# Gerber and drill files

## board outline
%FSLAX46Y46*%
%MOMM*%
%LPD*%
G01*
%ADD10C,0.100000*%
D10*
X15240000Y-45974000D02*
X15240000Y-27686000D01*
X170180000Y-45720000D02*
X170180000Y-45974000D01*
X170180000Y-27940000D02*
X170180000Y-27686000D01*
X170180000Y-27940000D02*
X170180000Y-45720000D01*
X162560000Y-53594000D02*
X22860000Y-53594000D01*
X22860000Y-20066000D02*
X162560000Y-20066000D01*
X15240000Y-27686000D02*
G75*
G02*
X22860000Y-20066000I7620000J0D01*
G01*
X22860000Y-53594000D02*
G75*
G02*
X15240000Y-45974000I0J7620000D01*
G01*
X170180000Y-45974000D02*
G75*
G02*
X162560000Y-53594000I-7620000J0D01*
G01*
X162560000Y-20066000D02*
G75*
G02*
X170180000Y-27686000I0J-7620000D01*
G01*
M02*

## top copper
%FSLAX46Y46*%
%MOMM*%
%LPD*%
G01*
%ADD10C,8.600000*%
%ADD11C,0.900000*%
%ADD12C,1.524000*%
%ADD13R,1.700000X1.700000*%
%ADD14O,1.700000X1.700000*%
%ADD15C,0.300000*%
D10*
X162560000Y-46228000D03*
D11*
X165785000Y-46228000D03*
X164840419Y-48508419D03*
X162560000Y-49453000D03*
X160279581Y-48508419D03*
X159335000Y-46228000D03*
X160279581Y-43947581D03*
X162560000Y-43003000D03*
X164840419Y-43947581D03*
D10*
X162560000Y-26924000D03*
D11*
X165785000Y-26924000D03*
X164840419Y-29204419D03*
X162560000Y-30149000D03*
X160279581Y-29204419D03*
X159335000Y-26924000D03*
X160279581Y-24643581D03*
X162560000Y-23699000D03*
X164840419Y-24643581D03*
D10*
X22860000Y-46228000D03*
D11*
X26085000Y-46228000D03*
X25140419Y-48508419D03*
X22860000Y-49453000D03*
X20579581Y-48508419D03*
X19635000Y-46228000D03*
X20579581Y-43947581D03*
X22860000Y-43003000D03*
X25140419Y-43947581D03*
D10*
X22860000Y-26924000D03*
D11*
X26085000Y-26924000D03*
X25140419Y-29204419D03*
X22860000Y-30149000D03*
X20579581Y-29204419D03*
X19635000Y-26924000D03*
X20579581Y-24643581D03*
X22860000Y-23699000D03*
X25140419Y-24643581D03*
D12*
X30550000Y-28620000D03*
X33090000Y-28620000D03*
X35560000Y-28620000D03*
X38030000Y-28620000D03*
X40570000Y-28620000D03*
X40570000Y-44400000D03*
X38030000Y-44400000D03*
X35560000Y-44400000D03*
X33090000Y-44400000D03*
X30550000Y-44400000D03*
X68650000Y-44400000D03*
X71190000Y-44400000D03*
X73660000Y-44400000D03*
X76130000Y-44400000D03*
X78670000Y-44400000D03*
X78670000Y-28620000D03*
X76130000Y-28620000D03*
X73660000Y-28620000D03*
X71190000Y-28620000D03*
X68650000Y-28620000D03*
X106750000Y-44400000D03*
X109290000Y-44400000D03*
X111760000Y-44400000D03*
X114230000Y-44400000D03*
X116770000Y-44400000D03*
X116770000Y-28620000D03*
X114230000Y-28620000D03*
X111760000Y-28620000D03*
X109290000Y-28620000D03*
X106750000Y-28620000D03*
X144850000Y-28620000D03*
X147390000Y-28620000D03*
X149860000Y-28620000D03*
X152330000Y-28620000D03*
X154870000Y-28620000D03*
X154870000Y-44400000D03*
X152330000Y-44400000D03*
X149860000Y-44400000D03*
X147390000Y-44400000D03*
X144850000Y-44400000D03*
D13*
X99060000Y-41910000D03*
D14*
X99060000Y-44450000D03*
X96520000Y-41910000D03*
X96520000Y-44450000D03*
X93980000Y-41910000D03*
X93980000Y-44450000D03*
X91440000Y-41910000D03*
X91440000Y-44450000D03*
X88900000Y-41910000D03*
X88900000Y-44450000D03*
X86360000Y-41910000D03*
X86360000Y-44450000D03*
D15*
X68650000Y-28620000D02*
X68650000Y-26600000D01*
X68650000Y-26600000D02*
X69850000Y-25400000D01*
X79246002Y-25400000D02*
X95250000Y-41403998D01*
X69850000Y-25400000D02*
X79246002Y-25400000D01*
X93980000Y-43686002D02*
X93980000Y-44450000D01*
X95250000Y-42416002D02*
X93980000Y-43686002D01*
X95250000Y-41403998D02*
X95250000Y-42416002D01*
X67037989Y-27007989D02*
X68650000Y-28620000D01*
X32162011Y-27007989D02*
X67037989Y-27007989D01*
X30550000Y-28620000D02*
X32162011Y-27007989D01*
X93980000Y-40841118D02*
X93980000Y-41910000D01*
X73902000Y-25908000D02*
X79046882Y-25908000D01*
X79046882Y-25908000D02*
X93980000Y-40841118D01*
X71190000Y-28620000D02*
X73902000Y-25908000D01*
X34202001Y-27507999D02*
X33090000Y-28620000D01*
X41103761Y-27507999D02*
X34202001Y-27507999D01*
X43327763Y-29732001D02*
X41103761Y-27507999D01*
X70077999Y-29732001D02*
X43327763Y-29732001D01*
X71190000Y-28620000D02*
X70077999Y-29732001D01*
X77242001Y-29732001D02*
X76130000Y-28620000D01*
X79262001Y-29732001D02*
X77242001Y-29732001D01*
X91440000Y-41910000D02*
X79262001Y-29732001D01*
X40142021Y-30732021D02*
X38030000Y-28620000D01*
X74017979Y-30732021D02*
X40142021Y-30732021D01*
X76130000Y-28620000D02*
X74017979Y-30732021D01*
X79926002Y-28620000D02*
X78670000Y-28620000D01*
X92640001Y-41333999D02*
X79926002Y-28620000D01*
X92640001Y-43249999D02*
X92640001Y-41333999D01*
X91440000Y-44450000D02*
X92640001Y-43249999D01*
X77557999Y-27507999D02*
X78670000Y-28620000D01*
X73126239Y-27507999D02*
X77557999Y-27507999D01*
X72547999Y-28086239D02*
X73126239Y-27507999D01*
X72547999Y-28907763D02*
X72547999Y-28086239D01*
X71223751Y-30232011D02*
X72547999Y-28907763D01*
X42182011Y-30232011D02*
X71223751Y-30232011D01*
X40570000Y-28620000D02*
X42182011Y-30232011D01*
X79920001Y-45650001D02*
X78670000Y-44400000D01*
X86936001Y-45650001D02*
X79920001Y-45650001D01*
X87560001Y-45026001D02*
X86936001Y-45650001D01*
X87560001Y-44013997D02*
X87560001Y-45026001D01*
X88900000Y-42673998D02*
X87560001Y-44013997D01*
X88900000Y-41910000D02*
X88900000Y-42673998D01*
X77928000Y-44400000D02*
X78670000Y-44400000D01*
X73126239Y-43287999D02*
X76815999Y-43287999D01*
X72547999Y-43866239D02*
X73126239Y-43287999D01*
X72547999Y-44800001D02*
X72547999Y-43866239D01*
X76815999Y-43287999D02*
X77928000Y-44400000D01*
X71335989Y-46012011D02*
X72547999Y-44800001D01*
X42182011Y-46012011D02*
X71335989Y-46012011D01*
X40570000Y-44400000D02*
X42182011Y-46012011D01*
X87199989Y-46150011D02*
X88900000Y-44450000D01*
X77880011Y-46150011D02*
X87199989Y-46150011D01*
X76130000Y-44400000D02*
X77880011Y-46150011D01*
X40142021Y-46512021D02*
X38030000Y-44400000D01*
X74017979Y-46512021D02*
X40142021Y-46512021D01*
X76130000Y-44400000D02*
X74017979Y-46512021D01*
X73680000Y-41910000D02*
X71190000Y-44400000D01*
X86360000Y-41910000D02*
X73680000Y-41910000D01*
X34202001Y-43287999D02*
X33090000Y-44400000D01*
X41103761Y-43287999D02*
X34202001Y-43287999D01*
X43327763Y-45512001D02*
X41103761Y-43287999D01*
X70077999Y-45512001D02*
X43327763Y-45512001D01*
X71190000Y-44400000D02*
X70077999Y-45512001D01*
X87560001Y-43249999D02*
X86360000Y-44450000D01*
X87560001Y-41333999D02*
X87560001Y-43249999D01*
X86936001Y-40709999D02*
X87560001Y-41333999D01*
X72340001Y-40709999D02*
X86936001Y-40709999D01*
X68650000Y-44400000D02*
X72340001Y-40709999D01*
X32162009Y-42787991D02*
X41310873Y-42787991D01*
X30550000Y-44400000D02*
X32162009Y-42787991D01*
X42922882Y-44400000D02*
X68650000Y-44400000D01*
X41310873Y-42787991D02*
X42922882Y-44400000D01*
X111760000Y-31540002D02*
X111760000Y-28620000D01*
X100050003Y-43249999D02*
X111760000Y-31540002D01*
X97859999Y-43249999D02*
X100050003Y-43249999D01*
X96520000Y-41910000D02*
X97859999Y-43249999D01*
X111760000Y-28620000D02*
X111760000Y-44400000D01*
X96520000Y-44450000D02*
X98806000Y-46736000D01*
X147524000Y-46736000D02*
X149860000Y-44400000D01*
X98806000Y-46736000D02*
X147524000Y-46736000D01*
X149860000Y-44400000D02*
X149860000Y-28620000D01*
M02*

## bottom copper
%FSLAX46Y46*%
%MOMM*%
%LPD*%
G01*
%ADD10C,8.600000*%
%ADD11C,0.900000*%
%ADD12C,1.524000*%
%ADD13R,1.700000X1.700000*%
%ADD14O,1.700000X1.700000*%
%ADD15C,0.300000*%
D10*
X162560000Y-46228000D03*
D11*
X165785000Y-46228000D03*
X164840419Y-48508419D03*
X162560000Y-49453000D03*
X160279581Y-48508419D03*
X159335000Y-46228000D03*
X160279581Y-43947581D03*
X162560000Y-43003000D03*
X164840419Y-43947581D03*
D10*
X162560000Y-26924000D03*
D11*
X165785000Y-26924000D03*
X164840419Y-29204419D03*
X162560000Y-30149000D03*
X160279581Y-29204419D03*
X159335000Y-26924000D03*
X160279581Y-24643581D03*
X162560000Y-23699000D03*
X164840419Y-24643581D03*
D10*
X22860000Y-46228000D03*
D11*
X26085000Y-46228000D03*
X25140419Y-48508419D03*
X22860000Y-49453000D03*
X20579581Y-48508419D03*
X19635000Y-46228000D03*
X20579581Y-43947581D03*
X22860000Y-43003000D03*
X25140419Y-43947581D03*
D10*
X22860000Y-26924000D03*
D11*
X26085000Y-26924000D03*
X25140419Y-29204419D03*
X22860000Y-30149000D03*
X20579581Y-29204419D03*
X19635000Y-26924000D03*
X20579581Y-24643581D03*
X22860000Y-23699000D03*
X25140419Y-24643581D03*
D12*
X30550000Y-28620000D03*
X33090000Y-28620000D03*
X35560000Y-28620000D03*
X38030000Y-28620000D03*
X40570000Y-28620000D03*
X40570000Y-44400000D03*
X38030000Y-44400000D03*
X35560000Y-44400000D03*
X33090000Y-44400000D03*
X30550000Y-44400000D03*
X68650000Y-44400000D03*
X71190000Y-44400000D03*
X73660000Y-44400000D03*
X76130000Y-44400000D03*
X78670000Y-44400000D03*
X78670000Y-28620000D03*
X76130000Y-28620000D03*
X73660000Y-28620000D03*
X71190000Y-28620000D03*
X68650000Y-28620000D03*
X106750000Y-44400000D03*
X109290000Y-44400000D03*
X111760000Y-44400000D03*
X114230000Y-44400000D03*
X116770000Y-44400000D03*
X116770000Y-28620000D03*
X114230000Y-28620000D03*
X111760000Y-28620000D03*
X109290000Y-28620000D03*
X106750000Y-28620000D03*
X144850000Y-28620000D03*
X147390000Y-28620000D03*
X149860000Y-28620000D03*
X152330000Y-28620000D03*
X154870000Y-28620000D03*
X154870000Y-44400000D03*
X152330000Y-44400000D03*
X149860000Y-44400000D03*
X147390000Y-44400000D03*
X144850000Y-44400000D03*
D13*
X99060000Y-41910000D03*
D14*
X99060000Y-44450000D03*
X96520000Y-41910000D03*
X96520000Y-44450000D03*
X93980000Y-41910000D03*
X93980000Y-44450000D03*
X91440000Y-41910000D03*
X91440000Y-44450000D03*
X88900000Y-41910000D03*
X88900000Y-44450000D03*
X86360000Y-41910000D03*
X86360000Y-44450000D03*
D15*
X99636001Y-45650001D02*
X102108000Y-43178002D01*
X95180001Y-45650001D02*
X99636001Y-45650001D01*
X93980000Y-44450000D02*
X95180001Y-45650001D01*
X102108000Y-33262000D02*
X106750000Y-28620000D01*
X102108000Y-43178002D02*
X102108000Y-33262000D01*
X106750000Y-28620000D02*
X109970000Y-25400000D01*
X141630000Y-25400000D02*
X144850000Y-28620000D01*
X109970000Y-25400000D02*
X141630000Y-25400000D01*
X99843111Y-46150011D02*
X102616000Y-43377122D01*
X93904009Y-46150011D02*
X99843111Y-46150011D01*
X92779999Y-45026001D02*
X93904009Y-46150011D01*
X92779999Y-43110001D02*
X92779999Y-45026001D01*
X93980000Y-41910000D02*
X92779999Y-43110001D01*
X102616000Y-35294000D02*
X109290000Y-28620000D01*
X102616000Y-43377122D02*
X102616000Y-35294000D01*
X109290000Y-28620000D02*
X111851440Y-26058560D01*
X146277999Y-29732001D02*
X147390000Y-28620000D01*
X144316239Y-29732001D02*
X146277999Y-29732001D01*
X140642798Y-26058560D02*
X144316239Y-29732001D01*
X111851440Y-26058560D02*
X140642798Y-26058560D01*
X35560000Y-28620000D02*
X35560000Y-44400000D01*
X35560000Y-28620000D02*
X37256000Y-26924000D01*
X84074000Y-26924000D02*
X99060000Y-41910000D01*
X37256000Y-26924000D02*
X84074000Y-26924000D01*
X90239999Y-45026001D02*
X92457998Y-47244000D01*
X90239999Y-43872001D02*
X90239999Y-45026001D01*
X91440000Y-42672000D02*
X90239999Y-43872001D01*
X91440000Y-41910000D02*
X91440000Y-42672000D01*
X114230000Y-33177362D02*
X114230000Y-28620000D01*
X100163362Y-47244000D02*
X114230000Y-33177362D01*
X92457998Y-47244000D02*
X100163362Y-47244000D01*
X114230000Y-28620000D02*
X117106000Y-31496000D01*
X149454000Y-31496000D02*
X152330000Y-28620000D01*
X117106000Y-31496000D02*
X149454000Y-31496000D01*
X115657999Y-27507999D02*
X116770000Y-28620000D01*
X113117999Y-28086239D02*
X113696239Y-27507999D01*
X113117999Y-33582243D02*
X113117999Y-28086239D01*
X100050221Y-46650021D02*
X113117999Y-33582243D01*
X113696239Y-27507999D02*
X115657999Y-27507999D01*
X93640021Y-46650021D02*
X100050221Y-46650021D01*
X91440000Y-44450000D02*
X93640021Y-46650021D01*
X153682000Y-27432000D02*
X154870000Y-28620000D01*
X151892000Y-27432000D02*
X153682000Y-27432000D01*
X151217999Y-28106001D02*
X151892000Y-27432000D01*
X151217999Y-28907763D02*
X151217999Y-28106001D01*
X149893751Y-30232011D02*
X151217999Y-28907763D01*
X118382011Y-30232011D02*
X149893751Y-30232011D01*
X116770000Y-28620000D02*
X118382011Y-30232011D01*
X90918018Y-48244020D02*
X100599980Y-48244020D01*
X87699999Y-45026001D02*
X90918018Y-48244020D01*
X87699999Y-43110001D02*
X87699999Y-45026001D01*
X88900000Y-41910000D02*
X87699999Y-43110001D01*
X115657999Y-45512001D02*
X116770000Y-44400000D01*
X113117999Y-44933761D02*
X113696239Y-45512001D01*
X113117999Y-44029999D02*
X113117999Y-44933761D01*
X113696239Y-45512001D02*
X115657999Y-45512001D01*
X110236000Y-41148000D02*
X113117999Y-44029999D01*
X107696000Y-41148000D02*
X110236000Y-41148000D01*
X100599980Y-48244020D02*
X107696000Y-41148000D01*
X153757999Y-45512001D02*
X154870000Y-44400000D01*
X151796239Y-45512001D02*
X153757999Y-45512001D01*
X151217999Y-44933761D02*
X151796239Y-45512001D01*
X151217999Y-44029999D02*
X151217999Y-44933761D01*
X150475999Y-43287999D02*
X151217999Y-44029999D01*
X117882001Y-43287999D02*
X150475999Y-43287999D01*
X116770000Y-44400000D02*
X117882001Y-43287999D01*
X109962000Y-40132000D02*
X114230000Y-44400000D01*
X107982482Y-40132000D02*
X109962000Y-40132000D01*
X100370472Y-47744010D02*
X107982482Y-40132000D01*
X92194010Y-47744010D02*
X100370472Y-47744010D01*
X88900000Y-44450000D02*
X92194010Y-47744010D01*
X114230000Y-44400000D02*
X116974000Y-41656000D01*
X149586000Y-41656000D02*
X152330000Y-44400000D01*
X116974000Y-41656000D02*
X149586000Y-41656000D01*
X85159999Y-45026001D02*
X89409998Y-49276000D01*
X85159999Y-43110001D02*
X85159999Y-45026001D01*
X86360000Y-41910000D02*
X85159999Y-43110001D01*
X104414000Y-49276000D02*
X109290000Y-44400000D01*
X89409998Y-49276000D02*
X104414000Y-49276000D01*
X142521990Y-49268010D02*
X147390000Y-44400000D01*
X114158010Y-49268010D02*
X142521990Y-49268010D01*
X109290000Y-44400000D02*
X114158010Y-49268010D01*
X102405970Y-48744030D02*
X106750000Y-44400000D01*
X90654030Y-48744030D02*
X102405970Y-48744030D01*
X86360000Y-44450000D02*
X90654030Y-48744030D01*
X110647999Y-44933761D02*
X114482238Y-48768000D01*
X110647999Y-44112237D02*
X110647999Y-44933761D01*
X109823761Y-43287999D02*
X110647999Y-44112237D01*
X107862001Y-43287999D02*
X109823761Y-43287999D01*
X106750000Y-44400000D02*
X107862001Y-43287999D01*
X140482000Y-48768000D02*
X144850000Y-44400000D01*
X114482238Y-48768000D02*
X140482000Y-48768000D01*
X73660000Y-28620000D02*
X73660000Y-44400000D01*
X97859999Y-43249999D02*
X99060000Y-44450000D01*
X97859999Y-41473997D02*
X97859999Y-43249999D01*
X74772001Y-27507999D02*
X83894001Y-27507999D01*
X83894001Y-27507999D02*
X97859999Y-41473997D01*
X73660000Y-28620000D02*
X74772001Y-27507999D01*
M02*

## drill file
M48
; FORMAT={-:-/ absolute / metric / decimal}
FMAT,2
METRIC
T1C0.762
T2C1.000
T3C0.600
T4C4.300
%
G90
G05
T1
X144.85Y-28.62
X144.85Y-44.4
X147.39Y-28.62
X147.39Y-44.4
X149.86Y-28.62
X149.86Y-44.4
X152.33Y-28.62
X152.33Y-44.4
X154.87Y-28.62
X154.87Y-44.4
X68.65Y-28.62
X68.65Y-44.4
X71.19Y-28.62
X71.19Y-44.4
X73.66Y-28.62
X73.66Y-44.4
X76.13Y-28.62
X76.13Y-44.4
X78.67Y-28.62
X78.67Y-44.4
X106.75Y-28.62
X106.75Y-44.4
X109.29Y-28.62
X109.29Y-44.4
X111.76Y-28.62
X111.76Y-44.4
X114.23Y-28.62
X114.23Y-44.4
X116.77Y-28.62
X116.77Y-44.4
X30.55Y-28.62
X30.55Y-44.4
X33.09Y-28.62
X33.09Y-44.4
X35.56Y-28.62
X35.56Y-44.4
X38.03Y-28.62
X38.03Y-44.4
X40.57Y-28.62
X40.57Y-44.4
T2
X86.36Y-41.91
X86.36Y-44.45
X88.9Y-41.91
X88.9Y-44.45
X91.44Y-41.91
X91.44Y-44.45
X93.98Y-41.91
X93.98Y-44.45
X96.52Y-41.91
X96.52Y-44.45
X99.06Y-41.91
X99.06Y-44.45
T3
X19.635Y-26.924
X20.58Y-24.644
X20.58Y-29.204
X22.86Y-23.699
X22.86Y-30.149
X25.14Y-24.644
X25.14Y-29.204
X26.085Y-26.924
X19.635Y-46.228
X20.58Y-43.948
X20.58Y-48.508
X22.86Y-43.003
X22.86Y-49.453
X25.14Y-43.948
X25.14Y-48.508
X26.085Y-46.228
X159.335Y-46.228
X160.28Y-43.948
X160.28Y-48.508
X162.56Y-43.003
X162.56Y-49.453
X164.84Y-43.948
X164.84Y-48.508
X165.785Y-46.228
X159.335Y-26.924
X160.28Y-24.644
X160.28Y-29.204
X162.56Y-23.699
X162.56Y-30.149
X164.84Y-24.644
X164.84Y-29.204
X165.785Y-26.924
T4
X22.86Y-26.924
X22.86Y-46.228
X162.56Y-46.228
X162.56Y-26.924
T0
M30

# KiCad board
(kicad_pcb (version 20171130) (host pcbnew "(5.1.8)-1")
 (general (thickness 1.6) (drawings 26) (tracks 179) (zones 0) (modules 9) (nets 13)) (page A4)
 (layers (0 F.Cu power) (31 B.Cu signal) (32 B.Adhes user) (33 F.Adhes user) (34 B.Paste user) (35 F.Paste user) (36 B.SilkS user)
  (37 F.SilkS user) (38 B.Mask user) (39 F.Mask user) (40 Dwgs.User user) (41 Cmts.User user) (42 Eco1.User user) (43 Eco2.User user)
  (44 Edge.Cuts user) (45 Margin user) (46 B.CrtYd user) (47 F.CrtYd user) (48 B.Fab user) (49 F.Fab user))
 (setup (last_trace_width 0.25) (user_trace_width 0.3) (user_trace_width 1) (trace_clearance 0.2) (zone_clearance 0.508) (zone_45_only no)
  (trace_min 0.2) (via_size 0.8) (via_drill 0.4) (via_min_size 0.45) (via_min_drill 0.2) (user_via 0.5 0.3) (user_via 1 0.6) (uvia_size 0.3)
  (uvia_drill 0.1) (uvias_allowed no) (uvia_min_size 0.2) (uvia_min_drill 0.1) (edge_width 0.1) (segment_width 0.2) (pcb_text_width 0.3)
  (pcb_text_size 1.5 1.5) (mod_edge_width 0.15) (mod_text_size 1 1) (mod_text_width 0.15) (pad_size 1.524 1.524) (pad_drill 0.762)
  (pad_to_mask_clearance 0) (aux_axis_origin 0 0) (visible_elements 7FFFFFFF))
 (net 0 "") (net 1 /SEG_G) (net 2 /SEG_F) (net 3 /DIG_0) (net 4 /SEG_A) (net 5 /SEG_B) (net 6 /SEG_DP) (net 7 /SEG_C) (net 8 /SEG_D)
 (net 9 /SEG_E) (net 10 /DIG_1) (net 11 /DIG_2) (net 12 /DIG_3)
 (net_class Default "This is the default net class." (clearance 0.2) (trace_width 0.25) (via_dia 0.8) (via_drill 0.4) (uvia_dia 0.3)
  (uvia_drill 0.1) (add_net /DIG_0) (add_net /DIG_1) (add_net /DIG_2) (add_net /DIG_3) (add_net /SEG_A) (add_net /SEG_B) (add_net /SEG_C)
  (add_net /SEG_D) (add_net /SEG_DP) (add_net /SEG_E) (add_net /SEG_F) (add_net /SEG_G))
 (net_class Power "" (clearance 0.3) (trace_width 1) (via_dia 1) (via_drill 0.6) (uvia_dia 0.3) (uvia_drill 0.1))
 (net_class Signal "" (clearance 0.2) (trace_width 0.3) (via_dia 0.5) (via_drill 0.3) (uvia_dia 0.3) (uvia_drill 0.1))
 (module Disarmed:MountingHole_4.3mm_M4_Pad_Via (layer F.Cu) (at 162.56 46.228)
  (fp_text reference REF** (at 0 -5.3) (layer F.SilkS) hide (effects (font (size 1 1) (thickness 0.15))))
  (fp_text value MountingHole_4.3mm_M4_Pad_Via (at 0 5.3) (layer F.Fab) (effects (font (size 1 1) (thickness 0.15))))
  (pad "" np_thru_hole circle (at 0 0) (size 8.6 8.6) (drill 4.3) (layers *.Cu *.Mask))
  (pad "" np_thru_hole circle (at 3.225 0) (size 0.9 0.9) (drill 0.6) (layers *.Cu *.Mask))
  (pad "" np_thru_hole circle (at 2.280419 2.280419) (size 0.9 0.9) (drill 0.6) (layers *.Cu *.Mask))
  (pad "" np_thru_hole circle (at 0 3.225) (size 0.9 0.9) (drill 0.6) (layers *.Cu *.Mask))
  (pad "" np_thru_hole circle (at -2.280419 2.280419) (size 0.9 0.9) (drill 0.6) (layers *.Cu *.Mask))
  (pad "" np_thru_hole circle (at -3.225 0) (size 0.9 0.9) (drill 0.6) (layers *.Cu *.Mask))
  (pad "" np_thru_hole circle (at -2.280419 -2.280419) (size 0.9 0.9) (drill 0.6) (layers *.Cu *.Mask))
  (pad "" np_thru_hole circle (at 0 -3.225) (size 0.9 0.9) (drill 0.6) (layers *.Cu *.Mask))
  (pad "" np_thru_hole circle (at 2.280419 -2.280419) (size 0.9 0.9) (drill 0.6) (layers *.Cu *.Mask)))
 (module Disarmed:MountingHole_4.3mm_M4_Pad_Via (layer F.Cu) (at 162.56 26.924)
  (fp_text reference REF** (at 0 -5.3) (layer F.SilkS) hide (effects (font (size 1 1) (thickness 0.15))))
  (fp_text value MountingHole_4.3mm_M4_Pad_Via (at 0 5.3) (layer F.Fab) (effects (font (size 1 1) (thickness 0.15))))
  (pad "" np_thru_hole circle (at 0 0) (size 8.6 8.6) (drill 4.3) (layers *.Cu *.Mask))
  (pad "" np_thru_hole circle (at 3.225 0) (size 0.9 0.9) (drill 0.6) (layers *.Cu *.Mask))
  (pad "" np_thru_hole circle (at 2.280419 2.280419) (size 0.9 0.9) (drill 0.6) (layers *.Cu *.Mask))
  (pad "" np_thru_hole circle (at 0 3.225) (size 0.9 0.9) (drill 0.6) (layers *.Cu *.Mask))
  (pad "" np_thru_hole circle (at -2.280419 2.280419) (size 0.9 0.9) (drill 0.6) (layers *.Cu *.Mask))
  (pad "" np_thru_hole circle (at -3.225 0) (size 0.9 0.9) (drill 0.6) (layers *.Cu *.Mask))
  (pad "" np_thru_hole circle (at -2.280419 -2.280419) (size 0.9 0.9) (drill 0.6) (layers *.Cu *.Mask))
  (pad "" np_thru_hole circle (at 0 -3.225) (size 0.9 0.9) (drill 0.6) (layers *.Cu *.Mask))
  (pad "" np_thru_hole circle (at 2.280419 -2.280419) (size 0.9 0.9) (drill 0.6) (layers *.Cu *.Mask)))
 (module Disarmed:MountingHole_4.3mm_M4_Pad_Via (layer F.Cu) (at 22.86 46.228)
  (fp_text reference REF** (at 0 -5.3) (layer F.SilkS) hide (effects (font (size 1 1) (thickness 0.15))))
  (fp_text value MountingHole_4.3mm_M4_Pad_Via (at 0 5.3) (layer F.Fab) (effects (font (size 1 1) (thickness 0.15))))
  (pad "" np_thru_hole circle (at 0 0) (size 8.6 8.6) (drill 4.3) (layers *.Cu *.Mask))
  (pad "" np_thru_hole circle (at 3.225 0) (size 0.9 0.9) (drill 0.6) (layers *.Cu *.Mask))
  (pad "" np_thru_hole circle (at 2.280419 2.280419) (size 0.9 0.9) (drill 0.6) (layers *.Cu *.Mask))
  (pad "" np_thru_hole circle (at 0 3.225) (size 0.9 0.9) (drill 0.6) (layers *.Cu *.Mask))
  (pad "" np_thru_hole circle (at -2.280419 2.280419) (size 0.9 0.9) (drill 0.6) (layers *.Cu *.Mask))
  (pad "" np_thru_hole circle (at -3.225 0) (size 0.9 0.9) (drill 0.6) (layers *.Cu *.Mask))
  (pad "" np_thru_hole circle (at -2.280419 -2.280419) (size 0.9 0.9) (drill 0.6) (layers *.Cu *.Mask))
  (pad "" np_thru_hole circle (at 0 -3.225) (size 0.9 0.9) (drill 0.6) (layers *.Cu *.Mask))
  (pad "" np_thru_hole circle (at 2.280419 -2.280419) (size 0.9 0.9) (drill 0.6) (layers *.Cu *.Mask)))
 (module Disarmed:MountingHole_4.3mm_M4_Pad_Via (layer F.Cu) (at 22.86 26.924)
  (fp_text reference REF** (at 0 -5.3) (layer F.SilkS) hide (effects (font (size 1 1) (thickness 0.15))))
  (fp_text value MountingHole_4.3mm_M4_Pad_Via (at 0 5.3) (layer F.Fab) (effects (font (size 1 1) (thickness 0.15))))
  (pad "" np_thru_hole circle (at 0 0) (size 8.6 8.6) (drill 4.3) (layers *.Cu *.Mask))
  (pad "" np_thru_hole circle (at 3.225 0) (size 0.9 0.9) (drill 0.6) (layers *.Cu *.Mask))
  (pad "" np_thru_hole circle (at 2.280419 2.280419) (size 0.9 0.9) (drill 0.6) (layers *.Cu *.Mask))
  (pad "" np_thru_hole circle (at 0 3.225) (size 0.9 0.9) (drill 0.6) (layers *.Cu *.Mask))
  (pad "" np_thru_hole circle (at -2.280419 2.280419) (size 0.9 0.9) (drill 0.6) (layers *.Cu *.Mask))
  (pad "" np_thru_hole circle (at -3.225 0) (size 0.9 0.9) (drill 0.6) (layers *.Cu *.Mask))
  (pad "" np_thru_hole circle (at -2.280419 -2.280419) (size 0.9 0.9) (drill 0.6) (layers *.Cu *.Mask))
  (pad "" np_thru_hole circle (at 0 -3.225) (size 0.9 0.9) (drill 0.6) (layers *.Cu *.Mask))
  (pad "" np_thru_hole circle (at 2.280419 -2.280419) (size 0.9 0.9) (drill 0.6) (layers *.Cu *.Mask)))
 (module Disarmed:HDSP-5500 (layer F.Cu) (at 35.56 36.83)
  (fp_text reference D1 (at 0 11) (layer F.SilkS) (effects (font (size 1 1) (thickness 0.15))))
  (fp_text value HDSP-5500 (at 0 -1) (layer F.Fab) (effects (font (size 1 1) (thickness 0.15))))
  (pad 10 thru_hole circle (at -5.01 -8.21) (size 1.524 1.524) (drill 0.762) (layers *.Cu *.Mask) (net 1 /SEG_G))
  (pad 9 thru_hole circle (at -2.47 -8.21) (size 1.524 1.524) (drill 0.762) (layers *.Cu *.Mask) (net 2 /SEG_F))
  (pad 8 thru_hole circle (at 0 -8.21) (size 1.524 1.524) (drill 0.762) (layers *.Cu *.Mask) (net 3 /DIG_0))
  (pad 7 thru_hole circle (at 2.47 -8.21) (size 1.524 1.524) (drill 0.762) (layers *.Cu *.Mask) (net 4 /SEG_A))
  (pad 6 thru_hole circle (at 5.01 -8.21) (size 1.524 1.524) (drill 0.762) (layers *.Cu *.Mask) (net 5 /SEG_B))
  (pad 5 thru_hole circle (at 5.01 7.57) (size 1.524 1.524) (drill 0.762) (layers *.Cu *.Mask) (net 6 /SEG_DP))
  (pad 4 thru_hole circle (at 2.47 7.57) (size 1.524 1.524) (drill 0.762) (layers *.Cu *.Mask) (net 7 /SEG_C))
  (pad 3 thru_hole circle (at 0 7.57) (size 1.524 1.524) (drill 0.762) (layers *.Cu *.Mask) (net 3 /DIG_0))
  (pad 2 thru_hole circle (at -2.47 7.57) (size 1.524 1.524) (drill 0.762) (layers *.Cu *.Mask) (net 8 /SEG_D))
  (pad 1 thru_hole circle (at -5.01 7.57) (size 1.524 1.524) (drill 0.762) (layers *.Cu *.Mask) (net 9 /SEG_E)))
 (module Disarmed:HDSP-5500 (layer F.Cu) (at 73.66 36.83)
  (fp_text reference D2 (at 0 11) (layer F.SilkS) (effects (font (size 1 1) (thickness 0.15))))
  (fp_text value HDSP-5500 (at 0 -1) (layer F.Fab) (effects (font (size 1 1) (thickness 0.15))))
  (pad 1 thru_hole circle (at -5.01 7.57) (size 1.524 1.524) (drill 0.762) (layers *.Cu *.Mask) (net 9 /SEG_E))
  (pad 2 thru_hole circle (at -2.47 7.57) (size 1.524 1.524) (drill 0.762) (layers *.Cu *.Mask) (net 8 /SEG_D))
  (pad 3 thru_hole circle (at 0 7.57) (size 1.524 1.524) (drill 0.762) (layers *.Cu *.Mask) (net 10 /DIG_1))
  (pad 4 thru_hole circle (at 2.47 7.57) (size 1.524 1.524) (drill 0.762) (layers *.Cu *.Mask) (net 7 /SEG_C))
  (pad 5 thru_hole circle (at 5.01 7.57) (size 1.524 1.524) (drill 0.762) (layers *.Cu *.Mask) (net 6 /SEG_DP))
  (pad 6 thru_hole circle (at 5.01 -8.21) (size 1.524 1.524) (drill 0.762) (layers *.Cu *.Mask) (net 5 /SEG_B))
  (pad 7 thru_hole circle (at 2.47 -8.21) (size 1.524 1.524) (drill 0.762) (layers *.Cu *.Mask) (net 4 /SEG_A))
  (pad 8 thru_hole circle (at 0 -8.21) (size 1.524 1.524) (drill 0.762) (layers *.Cu *.Mask) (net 10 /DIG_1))
  (pad 9 thru_hole circle (at -2.47 -8.21) (size 1.524 1.524) (drill 0.762) (layers *.Cu *.Mask) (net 2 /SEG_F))
  (pad 10 thru_hole circle (at -5.01 -8.21) (size 1.524 1.524) (drill 0.762) (layers *.Cu *.Mask) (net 1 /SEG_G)))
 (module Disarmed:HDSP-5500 (layer F.Cu) (at 111.76 36.83)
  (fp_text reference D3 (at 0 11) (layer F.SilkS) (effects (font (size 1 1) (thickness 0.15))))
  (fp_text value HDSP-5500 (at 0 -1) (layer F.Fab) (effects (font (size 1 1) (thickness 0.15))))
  (pad 1 thru_hole circle (at -5.01 7.57) (size 1.524 1.524) (drill 0.762) (layers *.Cu *.Mask) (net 9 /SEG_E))
  (pad 2 thru_hole circle (at -2.47 7.57) (size 1.524 1.524) (drill 0.762) (layers *.Cu *.Mask) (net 8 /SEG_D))
  (pad 3 thru_hole circle (at 0 7.57) (size 1.524 1.524) (drill 0.762) (layers *.Cu *.Mask) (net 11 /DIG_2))
  (pad 4 thru_hole circle (at 2.47 7.57) (size 1.524 1.524) (drill 0.762) (layers *.Cu *.Mask) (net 7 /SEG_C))
  (pad 5 thru_hole circle (at 5.01 7.57) (size 1.524 1.524) (drill 0.762) (layers *.Cu *.Mask) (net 6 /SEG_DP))
  (pad 6 thru_hole circle (at 5.01 -8.21) (size 1.524 1.524) (drill 0.762) (layers *.Cu *.Mask) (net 5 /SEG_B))
  (pad 7 thru_hole circle (at 2.47 -8.21) (size 1.524 1.524) (drill 0.762) (layers *.Cu *.Mask) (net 4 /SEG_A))
  (pad 8 thru_hole circle (at 0 -8.21) (size 1.524 1.524) (drill 0.762) (layers *.Cu *.Mask) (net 11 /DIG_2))
  (pad 9 thru_hole circle (at -2.47 -8.21) (size 1.524 1.524) (drill 0.762) (layers *.Cu *.Mask) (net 2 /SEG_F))
  (pad 10 thru_hole circle (at -5.01 -8.21) (size 1.524 1.524) (drill 0.762) (layers *.Cu *.Mask) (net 1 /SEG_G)))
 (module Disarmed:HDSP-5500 (layer F.Cu) (at 149.86 36.83)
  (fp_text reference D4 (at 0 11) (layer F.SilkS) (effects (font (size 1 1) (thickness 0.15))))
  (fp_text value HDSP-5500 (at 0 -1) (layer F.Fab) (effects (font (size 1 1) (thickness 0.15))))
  (pad 10 thru_hole circle (at -5.01 -8.21) (size 1.524 1.524) (drill 0.762) (layers *.Cu *.Mask) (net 1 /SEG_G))
  (pad 9 thru_hole circle (at -2.47 -8.21) (size 1.524 1.524) (drill 0.762) (layers *.Cu *.Mask) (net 2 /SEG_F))
  (pad 8 thru_hole circle (at 0 -8.21) (size 1.524 1.524) (drill 0.762) (layers *.Cu *.Mask) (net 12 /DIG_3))
  (pad 7 thru_hole circle (at 2.47 -8.21) (size 1.524 1.524) (drill 0.762) (layers *.Cu *.Mask) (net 4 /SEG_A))
  (pad 6 thru_hole circle (at 5.01 -8.21) (size 1.524 1.524) (drill 0.762) (layers *.Cu *.Mask) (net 5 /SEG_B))
  (pad 5 thru_hole circle (at 5.01 7.57) (size 1.524 1.524) (drill 0.762) (layers *.Cu *.Mask) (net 6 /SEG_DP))
  (pad 4 thru_hole circle (at 2.47 7.57) (size 1.524 1.524) (drill 0.762) (layers *.Cu *.Mask) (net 7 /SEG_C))
  (pad 3 thru_hole circle (at 0 7.57) (size 1.524 1.524) (drill 0.762) (layers *.Cu *.Mask) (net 12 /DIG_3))
  (pad 2 thru_hole circle (at -2.47 7.57) (size 1.524 1.524) (drill 0.762) (layers *.Cu *.Mask) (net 8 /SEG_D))
  (pad 1 thru_hole circle (at -5.01 7.57) (size 1.524 1.524) (drill 0.762) (layers *.Cu *.Mask) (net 9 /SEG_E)))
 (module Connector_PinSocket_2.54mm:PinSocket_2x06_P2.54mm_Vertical (layer B.Cu) (at 99.06 41.91 90)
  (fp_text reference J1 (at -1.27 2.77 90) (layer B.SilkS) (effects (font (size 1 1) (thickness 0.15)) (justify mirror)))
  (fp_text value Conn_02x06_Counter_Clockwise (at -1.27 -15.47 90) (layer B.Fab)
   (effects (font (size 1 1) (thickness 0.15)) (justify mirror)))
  (pad 1 thru_hole rect (at 0 0 90) (size 1.7 1.7) (drill 1) (layers *.Cu *.Mask) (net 3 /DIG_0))
  (pad 2 thru_hole oval (at -2.54 0 90) (size 1.7 1.7) (drill 1) (layers *.Cu *.Mask) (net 10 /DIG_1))
  (pad 3 thru_hole oval (at 0 -2.54 90) (size 1.7 1.7) (drill 1) (layers *.Cu *.Mask) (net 11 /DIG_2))
  (pad 4 thru_hole oval (at -2.54 -2.54 90) (size 1.7 1.7) (drill 1) (layers *.Cu *.Mask) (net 12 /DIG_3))
  (pad 5 thru_hole oval (at 0 -5.08 90) (size 1.7 1.7) (drill 1) (layers *.Cu *.Mask) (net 2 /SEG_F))
  (pad 6 thru_hole oval (at -2.54 -5.08 90) (size 1.7 1.7) (drill 1) (layers *.Cu *.Mask) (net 1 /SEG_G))
  (pad 7 thru_hole oval (at 0 -7.62 90) (size 1.7 1.7) (drill 1) (layers *.Cu *.Mask) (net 4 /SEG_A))
  (pad 8 thru_hole oval (at -2.54 -7.62 90) (size 1.7 1.7) (drill 1) (layers *.Cu *.Mask) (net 5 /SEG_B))
  (pad 9 thru_hole oval (at 0 -10.16 90) (size 1.7 1.7) (drill 1) (layers *.Cu *.Mask) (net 6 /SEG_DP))
  (pad 10 thru_hole oval (at -2.54 -10.16 90) (size 1.7 1.7) (drill 1) (layers *.Cu *.Mask) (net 7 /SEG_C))
  (pad 11 thru_hole oval (at 0 -12.7 90) (size 1.7 1.7) (drill 1) (layers *.Cu *.Mask) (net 8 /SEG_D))
  (pad 12 thru_hole oval (at -2.54 -12.7 90) (size 1.7 1.7) (drill 1) (layers *.Cu *.Mask) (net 9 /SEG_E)))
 (gr_line (start 15.24 45.974) (end 15.24 27.686) (layer Edge.Cuts) (width 0.1))
 (gr_line (start 170.18 45.72) (end 170.18 45.974) (layer Edge.Cuts) (width 0.1))
 (gr_line (start 170.18 27.94) (end 170.18 27.686) (layer Edge.Cuts) (width 0.1))
 (gr_line (start 170.18 27.94) (end 170.18 45.72) (layer Edge.Cuts) (width 0.1))
 (gr_line (start 162.56 53.594) (end 22.86 53.594) (layer Edge.Cuts) (width 0.1))
 (gr_line (start 22.86 20.066) (end 162.56 20.066) (layer Edge.Cuts) (width 0.1))
 (gr_arc (start 22.86 27.686) (end 22.86 20.066) (angle -90) (layer Edge.Cuts) (width 0.1))
 (gr_arc (start 22.86 45.974) (end 15.24 45.974) (angle -90) (layer Edge.Cuts) (width 0.1))
 (gr_arc (start 162.56 45.974) (end 162.56 53.594) (angle -90) (layer Edge.Cuts) (width 0.1))
 (gr_arc (start 162.56 27.686) (end 170.18 27.686) (angle -90) (layer Edge.Cuts) (width 0.1))
 (segment (start 68.65 28.62) (end 68.65 26.6) (width 0.3) (layer F.Cu) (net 1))
 (segment (start 68.65 26.6) (end 69.85 25.4) (width 0.3) (layer F.Cu) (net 1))
 (segment (start 79.246002 25.4) (end 95.25 41.403998) (width 0.3) (layer F.Cu) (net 1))
 (segment (start 69.85 25.4) (end 79.246002 25.4) (width 0.3) (layer F.Cu) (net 1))
 (segment (start 93.98 43.686002) (end 93.98 44.45) (width 0.3) (layer F.Cu) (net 1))
 (segment (start 95.25 42.416002) (end 93.98 43.686002) (width 0.3) (layer F.Cu) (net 1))
 (segment (start 95.25 41.403998) (end 95.25 42.416002) (width 0.3) (layer F.Cu) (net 1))
 (segment (start 67.037989 27.007989) (end 68.65 28.62) (width 0.3) (layer F.Cu) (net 1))
 (segment (start 32.162011 27.007989) (end 67.037989 27.007989) (width 0.3) (layer F.Cu) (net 1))
 (segment (start 30.55 28.62) (end 32.162011 27.007989) (width 0.3) (layer F.Cu) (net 1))
 (segment (start 99.636001 45.650001) (end 102.108 43.178002) (width 0.3) (layer B.Cu) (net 1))
 (segment (start 95.180001 45.650001) (end 99.636001 45.650001) (width 0.3) (layer B.Cu) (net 1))
 (segment (start 93.98 44.45) (end 95.180001 45.650001) (width 0.3) (layer B.Cu) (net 1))
 (segment (start 102.108 33.262) (end 106.75 28.62) (width 0.3) (layer B.Cu) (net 1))
 (segment (start 102.108 43.178002) (end 102.108 33.262) (width 0.3) (layer B.Cu) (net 1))
 (segment (start 106.75 28.62) (end 109.97 25.4) (width 0.3) (layer B.Cu) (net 1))
 (segment (start 141.63 25.4) (end 144.85 28.62) (width 0.3) (layer B.Cu) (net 1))
 (segment (start 109.97 25.4) (end 141.63 25.4) (width 0.3) (layer B.Cu) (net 1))
 (segment (start 93.98 40.841118) (end 93.98 41.91) (width 0.3) (layer F.Cu) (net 2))
 (segment (start 73.902 25.908) (end 79.046882 25.908) (width 0.3) (layer F.Cu) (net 2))
 (segment (start 79.046882 25.908) (end 93.98 40.841118) (width 0.3) (layer F.Cu) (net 2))
 (segment (start 71.19 28.62) (end 73.902 25.908) (width 0.3) (layer F.Cu) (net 2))
 (segment (start 34.202001 27.507999) (end 33.09 28.62) (width 0.3) (layer F.Cu) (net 2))
 (segment (start 41.103761 27.507999) (end 34.202001 27.507999) (width 0.3) (layer F.Cu) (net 2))
 (segment (start 43.327763 29.732001) (end 41.103761 27.507999) (width 0.3) (layer F.Cu) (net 2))
 (segment (start 70.077999 29.732001) (end 43.327763 29.732001) (width 0.3) (layer F.Cu) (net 2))
 (segment (start 71.19 28.62) (end 70.077999 29.732001) (width 0.3) (layer F.Cu) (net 2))
 (segment (start 99.843111 46.150011) (end 102.616 43.377122) (width 0.3) (layer B.Cu) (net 2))
 (segment (start 93.904009 46.150011) (end 99.843111 46.150011) (width 0.3) (layer B.Cu) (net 2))
 (segment (start 92.779999 45.026001) (end 93.904009 46.150011) (width 0.3) (layer B.Cu) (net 2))
 (segment (start 92.779999 43.110001) (end 92.779999 45.026001) (width 0.3) (layer B.Cu) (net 2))
 (segment (start 93.98 41.91) (end 92.779999 43.110001) (width 0.3) (layer B.Cu) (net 2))
 (segment (start 102.616 35.294) (end 109.29 28.62) (width 0.3) (layer B.Cu) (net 2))
 (segment (start 102.616 43.377122) (end 102.616 35.294) (width 0.3) (layer B.Cu) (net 2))
 (segment (start 109.29 28.62) (end 111.85144 26.05856) (width 0.3) (layer B.Cu) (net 2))
 (segment (start 146.277999 29.732001) (end 147.39 28.62) (width 0.3) (layer B.Cu) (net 2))
 (segment (start 144.316239 29.732001) (end 146.277999 29.732001) (width 0.3) (layer B.Cu) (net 2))
 (segment (start 140.642798 26.05856) (end 144.316239 29.732001) (width 0.3) (layer B.Cu) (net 2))
 (segment (start 111.85144 26.05856) (end 140.642798 26.05856) (width 0.3) (layer B.Cu) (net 2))
 (segment (start 35.56 28.62) (end 35.56 44.4) (width 0.3) (layer B.Cu) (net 3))
 (segment (start 35.56 28.62) (end 37.256 26.924) (width 0.3) (layer B.Cu) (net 3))
 (segment (start 84.074 26.924) (end 99.06 41.91) (width 0.3) (layer B.Cu) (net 3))
 (segment (start 37.256 26.924) (end 84.074 26.924) (width 0.3) (layer B.Cu) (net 3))
 (segment (start 77.242001 29.732001) (end 76.13 28.62) (width 0.3) (layer F.Cu) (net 4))
 (segment (start 79.262001 29.732001) (end 77.242001 29.732001) (width 0.3) (layer F.Cu) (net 4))
 (segment (start 91.44 41.91) (end 79.262001 29.732001) (width 0.3) (layer F.Cu) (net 4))
 (segment (start 40.142021 30.732021) (end 38.03 28.62) (width 0.3) (layer F.Cu) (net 4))
 (segment (start 74.017979 30.732021) (end 40.142021 30.732021) (width 0.3) (layer F.Cu) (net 4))
 (segment (start 76.13 28.62) (end 74.017979 30.732021) (width 0.3) (layer F.Cu) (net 4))
 (segment (start 90.239999 45.026001) (end 92.457998 47.244) (width 0.3) (layer B.Cu) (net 4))
 (segment (start 90.239999 43.872001) (end 90.239999 45.026001) (width 0.3) (layer B.Cu) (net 4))
 (segment (start 91.44 42.672) (end 90.239999 43.872001) (width 0.3) (layer B.Cu) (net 4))
 (segment (start 91.44 41.91) (end 91.44 42.672) (width 0.3) (layer B.Cu) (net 4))
 (segment (start 114.23 33.177362) (end 114.23 28.62) (width 0.3) (layer B.Cu) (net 4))
 (segment (start 100.163362 47.244) (end 114.23 33.177362) (width 0.3) (layer B.Cu) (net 4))
 (segment (start 92.457998 47.244) (end 100.163362 47.244) (width 0.3) (layer B.Cu) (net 4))
 (segment (start 114.23 28.62) (end 117.106 31.496) (width 0.3) (layer B.Cu) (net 4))
 (segment (start 149.454 31.496) (end 152.33 28.62) (width 0.3) (layer B.Cu) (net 4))
 (segment (start 117.106 31.496) (end 149.454 31.496) (width 0.3) (layer B.Cu) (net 4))
 (segment (start 79.926002 28.62) (end 78.67 28.62) (width 0.3) (layer F.Cu) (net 5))
 (segment (start 92.640001 41.333999) (end 79.926002 28.62) (width 0.3) (layer F.Cu) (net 5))
 (segment (start 92.640001 43.249999) (end 92.640001 41.333999) (width 0.3) (layer F.Cu) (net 5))
 (segment (start 91.44 44.45) (end 92.640001 43.249999) (width 0.3) (layer F.Cu) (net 5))
 (segment (start 77.557999 27.507999) (end 78.67 28.62) (width 0.3) (layer F.Cu) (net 5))
 (segment (start 73.126239 27.507999) (end 77.557999 27.507999) (width 0.3) (layer F.Cu) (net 5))
 (segment (start 72.547999 28.086239) (end 73.126239 27.507999) (width 0.3) (layer F.Cu) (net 5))
 (segment (start 72.547999 28.907763) (end 72.547999 28.086239) (width 0.3) (layer F.Cu) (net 5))
 (segment (start 71.223751 30.232011) (end 72.547999 28.907763) (width 0.3) (layer F.Cu) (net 5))
 (segment (start 42.182011 30.232011) (end 71.223751 30.232011) (width 0.3) (layer F.Cu) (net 5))
 (segment (start 40.57 28.62) (end 42.182011 30.232011) (width 0.3) (layer F.Cu) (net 5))
 (segment (start 115.657999 27.507999) (end 116.77 28.62) (width 0.3) (layer B.Cu) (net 5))
 (segment (start 113.117999 28.086239) (end 113.696239 27.507999) (width 0.3) (layer B.Cu) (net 5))
 (segment (start 113.117999 33.582243) (end 113.117999 28.086239) (width 0.3) (layer B.Cu) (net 5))
 (segment (start 100.050221 46.650021) (end 113.117999 33.582243) (width 0.3) (layer B.Cu) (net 5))
 (segment (start 113.696239 27.507999) (end 115.657999 27.507999) (width 0.3) (layer B.Cu) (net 5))
 (segment (start 93.640021 46.650021) (end 100.050221 46.650021) (width 0.3) (layer B.Cu) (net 5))
 (segment (start 91.44 44.45) (end 93.640021 46.650021) (width 0.3) (layer B.Cu) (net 5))
 (segment (start 153.682 27.432) (end 154.87 28.62) (width 0.3) (layer B.Cu) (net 5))
 (segment (start 151.892 27.432) (end 153.682 27.432) (width 0.3) (layer B.Cu) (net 5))
 (segment (start 151.217999 28.106001) (end 151.892 27.432) (width 0.3) (layer B.Cu) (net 5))
 (segment (start 151.217999 28.907763) (end 151.217999 28.106001) (width 0.3) (layer B.Cu) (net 5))
 (segment (start 149.893751 30.232011) (end 151.217999 28.907763) (width 0.3) (layer B.Cu) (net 5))
 (segment (start 118.382011 30.232011) (end 149.893751 30.232011) (width 0.3) (layer B.Cu) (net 5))
 (segment (start 116.77 28.62) (end 118.382011 30.232011) (width 0.3) (layer B.Cu) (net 5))
 (segment (start 79.920001 45.650001) (end 78.67 44.4) (width 0.3) (layer F.Cu) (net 6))
 (segment (start 86.936001 45.650001) (end 79.920001 45.650001) (width 0.3) (layer F.Cu) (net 6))
 (segment (start 87.560001 45.026001) (end 86.936001 45.650001) (width 0.3) (layer F.Cu) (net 6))
 (segment (start 87.560001 44.013997) (end 87.560001 45.026001) (width 0.3) (layer F.Cu) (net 6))
 (segment (start 88.9 42.673998) (end 87.560001 44.013997) (width 0.3) (layer F.Cu) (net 6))
 (segment (start 88.9 41.91) (end 88.9 42.673998) (width 0.3) (layer F.Cu) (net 6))
 (segment (start 77.928 44.4) (end 78.67 44.4) (width 0.3) (layer F.Cu) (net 6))
 (segment (start 73.126239 43.287999) (end 76.815999 43.287999) (width 0.3) (layer F.Cu) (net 6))
 (segment (start 72.547999 43.866239) (end 73.126239 43.287999) (width 0.3) (layer F.Cu) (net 6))
 (segment (start 72.547999 44.800001) (end 72.547999 43.866239) (width 0.3) (layer F.Cu) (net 6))
 (segment (start 76.815999 43.287999) (end 77.928 44.4) (width 0.3) (layer F.Cu) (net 6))
 (segment (start 71.335989 46.012011) (end 72.547999 44.800001) (width 0.3) (layer F.Cu) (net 6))
 (segment (start 42.182011 46.012011) (end 71.335989 46.012011) (width 0.3) (layer F.Cu) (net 6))
 (segment (start 40.57 44.4) (end 42.182011 46.012011) (width 0.3) (layer F.Cu) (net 6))
 (segment (start 90.918018 48.24402) (end 100.59998 48.24402) (width 0.3) (layer B.Cu) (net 6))
 (segment (start 87.699999 45.026001) (end 90.918018 48.24402) (width 0.3) (layer B.Cu) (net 6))
 (segment (start 87.699999 43.110001) (end 87.699999 45.026001) (width 0.3) (layer B.Cu) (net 6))
 (segment (start 88.9 41.91) (end 87.699999 43.110001) (width 0.3) (layer B.Cu) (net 6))
 (segment (start 115.657999 45.512001) (end 116.77 44.4) (width 0.3) (layer B.Cu) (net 6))
 (segment (start 113.117999 44.933761) (end 113.696239 45.512001) (width 0.3) (layer B.Cu) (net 6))
 (segment (start 113.117999 44.029999) (end 113.117999 44.933761) (width 0.3) (layer B.Cu) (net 6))
 (segment (start 113.696239 45.512001) (end 115.657999 45.512001) (width 0.3) (layer B.Cu) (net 6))
 (segment (start 110.236 41.148) (end 113.117999 44.029999) (width 0.3) (layer B.Cu) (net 6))
 (segment (start 107.696 41.148) (end 110.236 41.148) (width 0.3) (layer B.Cu) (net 6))
 (segment (start 100.59998 48.24402) (end 107.696 41.148) (width 0.3) (layer B.Cu) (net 6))
 (segment (start 153.757999 45.512001) (end 154.87 44.4) (width 0.3) (layer B.Cu) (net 6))
 (segment (start 151.796239 45.512001) (end 153.757999 45.512001) (width 0.3) (layer B.Cu) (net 6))
 (segment (start 151.217999 44.933761) (end 151.796239 45.512001) (width 0.3) (layer B.Cu) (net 6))
 (segment (start 151.217999 44.029999) (end 151.217999 44.933761) (width 0.3) (layer B.Cu) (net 6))
 (segment (start 150.475999 43.287999) (end 151.217999 44.029999) (width 0.3) (layer B.Cu) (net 6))
 (segment (start 117.882001 43.287999) (end 150.475999 43.287999) (width 0.3) (layer B.Cu) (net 6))
 (segment (start 116.77 44.4) (end 117.882001 43.287999) (width 0.3) (layer B.Cu) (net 6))
 (segment (start 87.199989 46.150011) (end 88.9 44.45) (width 0.3) (layer F.Cu) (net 7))
 (segment (start 77.880011 46.150011) (end 87.199989 46.150011) (width 0.3) (layer F.Cu) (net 7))
 (segment (start 76.13 44.4) (end 77.880011 46.150011) (width 0.3) (layer F.Cu) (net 7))
 (segment (start 40.142021 46.512021) (end 38.03 44.4) (width 0.3) (layer F.Cu) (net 7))
 (segment (start 74.017979 46.512021) (end 40.142021 46.512021) (width 0.3) (layer F.Cu) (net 7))
 (segment (start 76.13 44.4) (end 74.017979 46.512021) (width 0.3) (layer F.Cu) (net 7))
 (segment (start 109.962 40.132) (end 114.23 44.4) (width 0.3) (layer B.Cu) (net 7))
 (segment (start 107.982482 40.132) (end 109.962 40.132) (width 0.3) (layer B.Cu) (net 7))
 (segment (start 100.370472 47.74401) (end 107.982482 40.132) (width 0.3) (layer B.Cu) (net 7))
 (segment (start 92.19401 47.74401) (end 100.370472 47.74401) (width 0.3) (layer B.Cu) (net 7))
 (segment (start 88.9 44.45) (end 92.19401 47.74401) (width 0.3) (layer B.Cu) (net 7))
 (segment (start 114.23 44.4) (end 116.974 41.656) (width 0.3) (layer B.Cu) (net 7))
 (segment (start 149.586 41.656) (end 152.33 44.4) (width 0.3) (layer B.Cu) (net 7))
 (segment (start 116.974 41.656) (end 149.586 41.656) (width 0.3) (layer B.Cu) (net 7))
 (segment (start 73.68 41.91) (end 71.19 44.4) (width 0.3) (layer F.Cu) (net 8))
 (segment (start 86.36 41.91) (end 73.68 41.91) (width 0.3) (layer F.Cu) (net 8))
 (segment (start 34.202001 43.287999) (end 33.09 44.4) (width 0.3) (layer F.Cu) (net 8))
 (segment (start 41.103761 43.287999) (end 34.202001 43.287999) (width 0.3) (layer F.Cu) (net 8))
 (segment (start 43.327763 45.512001) (end 41.103761 43.287999) (width 0.3) (layer F.Cu) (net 8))
 (segment (start 70.077999 45.512001) (end 43.327763 45.512001) (width 0.3) (layer F.Cu) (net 8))
 (segment (start 71.19 44.4) (end 70.077999 45.512001) (width 0.3) (layer F.Cu) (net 8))
 (segment (start 85.159999 45.026001) (end 89.409998 49.276) (width 0.3) (layer B.Cu) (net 8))
 (segment (start 85.159999 43.110001) (end 85.159999 45.026001) (width 0.3) (layer B.Cu) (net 8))
 (segment (start 86.36 41.91) (end 85.159999 43.110001) (width 0.3) (layer B.Cu) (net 8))
 (segment (start 104.414 49.276) (end 109.29 44.4) (width 0.3) (layer B.Cu) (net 8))
 (segment (start 89.409998 49.276) (end 104.414 49.276) (width 0.3) (layer B.Cu) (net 8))
 (segment (start 142.52199 49.26801) (end 147.39 44.4) (width 0.3) (layer B.Cu) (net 8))
 (segment (start 114.15801 49.26801) (end 142.52199 49.26801) (width 0.3) (layer B.Cu) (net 8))
 (segment (start 109.29 44.4) (end 114.15801 49.26801) (width 0.3) (layer B.Cu) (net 8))
 (segment (start 87.560001 43.249999) (end 86.36 44.45) (width 0.3) (layer F.Cu) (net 9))
 (segment (start 87.560001 41.333999) (end 87.560001 43.249999) (width 0.3) (layer F.Cu) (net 9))
 (segment (start 86.936001 40.709999) (end 87.560001 41.333999) (width 0.3) (layer F.Cu) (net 9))
 (segment (start 72.340001 40.709999) (end 86.936001 40.709999) (width 0.3) (layer F.Cu) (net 9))
 (segment (start 68.65 44.4) (end 72.340001 40.709999) (width 0.3) (layer F.Cu) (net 9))
 (segment (start 32.162009 42.787991) (end 41.310873 42.787991) (width 0.3) (layer F.Cu) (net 9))
 (segment (start 30.55 44.4) (end 32.162009 42.787991) (width 0.3) (layer F.Cu) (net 9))
 (segment (start 42.922882 44.4) (end 68.65 44.4) (width 0.3) (layer F.Cu) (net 9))
 (segment (start 41.310873 42.787991) (end 42.922882 44.4) (width 0.3) (layer F.Cu) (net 9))
 (segment (start 102.40597 48.74403) (end 106.75 44.4) (width 0.3) (layer B.Cu) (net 9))
 (segment (start 90.65403 48.74403) (end 102.40597 48.74403) (width 0.3) (layer B.Cu) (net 9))
 (segment (start 86.36 44.45) (end 90.65403 48.74403) (width 0.3) (layer B.Cu) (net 9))
 (segment (start 110.647999 44.933761) (end 114.482238 48.768) (width 0.3) (layer B.Cu) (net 9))
 (segment (start 110.647999 44.112237) (end 110.647999 44.933761) (width 0.3) (layer B.Cu) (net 9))
 (segment (start 109.823761 43.287999) (end 110.647999 44.112237) (width 0.3) (layer B.Cu) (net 9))
 (segment (start 107.862001 43.287999) (end 109.823761 43.287999) (width 0.3) (layer B.Cu) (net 9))
 (segment (start 106.75 44.4) (end 107.862001 43.287999) (width 0.3) (layer B.Cu) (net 9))
 (segment (start 140.482 48.768) (end 144.85 44.4) (width 0.3) (layer B.Cu) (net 9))
 (segment (start 114.482238 48.768) (end 140.482 48.768) (width 0.3) (layer B.Cu) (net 9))
 (segment (start 73.66 28.62) (end 73.66 44.4) (width 0.3) (layer B.Cu) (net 10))
 (segment (start 97.859999 43.249999) (end 99.06 44.45) (width 0.3) (layer B.Cu) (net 10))
 (segment (start 97.859999 41.473997) (end 97.859999 43.249999) (width 0.3) (layer B.Cu) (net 10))
 (segment (start 74.772001 27.507999) (end 83.894001 27.507999) (width 0.3) (layer B.Cu) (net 10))
 (segment (start 83.894001 27.507999) (end 97.859999 41.473997) (width 0.3) (layer B.Cu) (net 10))
 (segment (start 73.66 28.62) (end 74.772001 27.507999) (width 0.3) (layer B.Cu) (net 10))
 (segment (start 111.76 31.540002) (end 111.76 28.62) (width 0.3) (layer F.Cu) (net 11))
 (segment (start 100.050003 43.249999) (end 111.76 31.540002) (width 0.3) (layer F.Cu) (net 11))
 (segment (start 97.859999 43.249999) (end 100.050003 43.249999) (width 0.3) (layer F.Cu) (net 11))
 (segment (start 96.52 41.91) (end 97.859999 43.249999) (width 0.3) (layer F.Cu) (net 11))
 (segment (start 111.76 28.62) (end 111.76 44.4) (width 0.3) (layer F.Cu) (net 11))
 (segment (start 96.52 44.45) (end 98.806 46.736) (width 0.3) (layer F.Cu) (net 12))
 (segment (start 147.524 46.736) (end 149.86 44.4) (width 0.3) (layer F.Cu) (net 12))
 (segment (start 98.806 46.736) (end 147.524 46.736) (width 0.3) (layer F.Cu) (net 12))
 (segment (start 149.86 44.4) (end 149.86 28.62) (width 0.3) (layer F.Cu) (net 12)))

